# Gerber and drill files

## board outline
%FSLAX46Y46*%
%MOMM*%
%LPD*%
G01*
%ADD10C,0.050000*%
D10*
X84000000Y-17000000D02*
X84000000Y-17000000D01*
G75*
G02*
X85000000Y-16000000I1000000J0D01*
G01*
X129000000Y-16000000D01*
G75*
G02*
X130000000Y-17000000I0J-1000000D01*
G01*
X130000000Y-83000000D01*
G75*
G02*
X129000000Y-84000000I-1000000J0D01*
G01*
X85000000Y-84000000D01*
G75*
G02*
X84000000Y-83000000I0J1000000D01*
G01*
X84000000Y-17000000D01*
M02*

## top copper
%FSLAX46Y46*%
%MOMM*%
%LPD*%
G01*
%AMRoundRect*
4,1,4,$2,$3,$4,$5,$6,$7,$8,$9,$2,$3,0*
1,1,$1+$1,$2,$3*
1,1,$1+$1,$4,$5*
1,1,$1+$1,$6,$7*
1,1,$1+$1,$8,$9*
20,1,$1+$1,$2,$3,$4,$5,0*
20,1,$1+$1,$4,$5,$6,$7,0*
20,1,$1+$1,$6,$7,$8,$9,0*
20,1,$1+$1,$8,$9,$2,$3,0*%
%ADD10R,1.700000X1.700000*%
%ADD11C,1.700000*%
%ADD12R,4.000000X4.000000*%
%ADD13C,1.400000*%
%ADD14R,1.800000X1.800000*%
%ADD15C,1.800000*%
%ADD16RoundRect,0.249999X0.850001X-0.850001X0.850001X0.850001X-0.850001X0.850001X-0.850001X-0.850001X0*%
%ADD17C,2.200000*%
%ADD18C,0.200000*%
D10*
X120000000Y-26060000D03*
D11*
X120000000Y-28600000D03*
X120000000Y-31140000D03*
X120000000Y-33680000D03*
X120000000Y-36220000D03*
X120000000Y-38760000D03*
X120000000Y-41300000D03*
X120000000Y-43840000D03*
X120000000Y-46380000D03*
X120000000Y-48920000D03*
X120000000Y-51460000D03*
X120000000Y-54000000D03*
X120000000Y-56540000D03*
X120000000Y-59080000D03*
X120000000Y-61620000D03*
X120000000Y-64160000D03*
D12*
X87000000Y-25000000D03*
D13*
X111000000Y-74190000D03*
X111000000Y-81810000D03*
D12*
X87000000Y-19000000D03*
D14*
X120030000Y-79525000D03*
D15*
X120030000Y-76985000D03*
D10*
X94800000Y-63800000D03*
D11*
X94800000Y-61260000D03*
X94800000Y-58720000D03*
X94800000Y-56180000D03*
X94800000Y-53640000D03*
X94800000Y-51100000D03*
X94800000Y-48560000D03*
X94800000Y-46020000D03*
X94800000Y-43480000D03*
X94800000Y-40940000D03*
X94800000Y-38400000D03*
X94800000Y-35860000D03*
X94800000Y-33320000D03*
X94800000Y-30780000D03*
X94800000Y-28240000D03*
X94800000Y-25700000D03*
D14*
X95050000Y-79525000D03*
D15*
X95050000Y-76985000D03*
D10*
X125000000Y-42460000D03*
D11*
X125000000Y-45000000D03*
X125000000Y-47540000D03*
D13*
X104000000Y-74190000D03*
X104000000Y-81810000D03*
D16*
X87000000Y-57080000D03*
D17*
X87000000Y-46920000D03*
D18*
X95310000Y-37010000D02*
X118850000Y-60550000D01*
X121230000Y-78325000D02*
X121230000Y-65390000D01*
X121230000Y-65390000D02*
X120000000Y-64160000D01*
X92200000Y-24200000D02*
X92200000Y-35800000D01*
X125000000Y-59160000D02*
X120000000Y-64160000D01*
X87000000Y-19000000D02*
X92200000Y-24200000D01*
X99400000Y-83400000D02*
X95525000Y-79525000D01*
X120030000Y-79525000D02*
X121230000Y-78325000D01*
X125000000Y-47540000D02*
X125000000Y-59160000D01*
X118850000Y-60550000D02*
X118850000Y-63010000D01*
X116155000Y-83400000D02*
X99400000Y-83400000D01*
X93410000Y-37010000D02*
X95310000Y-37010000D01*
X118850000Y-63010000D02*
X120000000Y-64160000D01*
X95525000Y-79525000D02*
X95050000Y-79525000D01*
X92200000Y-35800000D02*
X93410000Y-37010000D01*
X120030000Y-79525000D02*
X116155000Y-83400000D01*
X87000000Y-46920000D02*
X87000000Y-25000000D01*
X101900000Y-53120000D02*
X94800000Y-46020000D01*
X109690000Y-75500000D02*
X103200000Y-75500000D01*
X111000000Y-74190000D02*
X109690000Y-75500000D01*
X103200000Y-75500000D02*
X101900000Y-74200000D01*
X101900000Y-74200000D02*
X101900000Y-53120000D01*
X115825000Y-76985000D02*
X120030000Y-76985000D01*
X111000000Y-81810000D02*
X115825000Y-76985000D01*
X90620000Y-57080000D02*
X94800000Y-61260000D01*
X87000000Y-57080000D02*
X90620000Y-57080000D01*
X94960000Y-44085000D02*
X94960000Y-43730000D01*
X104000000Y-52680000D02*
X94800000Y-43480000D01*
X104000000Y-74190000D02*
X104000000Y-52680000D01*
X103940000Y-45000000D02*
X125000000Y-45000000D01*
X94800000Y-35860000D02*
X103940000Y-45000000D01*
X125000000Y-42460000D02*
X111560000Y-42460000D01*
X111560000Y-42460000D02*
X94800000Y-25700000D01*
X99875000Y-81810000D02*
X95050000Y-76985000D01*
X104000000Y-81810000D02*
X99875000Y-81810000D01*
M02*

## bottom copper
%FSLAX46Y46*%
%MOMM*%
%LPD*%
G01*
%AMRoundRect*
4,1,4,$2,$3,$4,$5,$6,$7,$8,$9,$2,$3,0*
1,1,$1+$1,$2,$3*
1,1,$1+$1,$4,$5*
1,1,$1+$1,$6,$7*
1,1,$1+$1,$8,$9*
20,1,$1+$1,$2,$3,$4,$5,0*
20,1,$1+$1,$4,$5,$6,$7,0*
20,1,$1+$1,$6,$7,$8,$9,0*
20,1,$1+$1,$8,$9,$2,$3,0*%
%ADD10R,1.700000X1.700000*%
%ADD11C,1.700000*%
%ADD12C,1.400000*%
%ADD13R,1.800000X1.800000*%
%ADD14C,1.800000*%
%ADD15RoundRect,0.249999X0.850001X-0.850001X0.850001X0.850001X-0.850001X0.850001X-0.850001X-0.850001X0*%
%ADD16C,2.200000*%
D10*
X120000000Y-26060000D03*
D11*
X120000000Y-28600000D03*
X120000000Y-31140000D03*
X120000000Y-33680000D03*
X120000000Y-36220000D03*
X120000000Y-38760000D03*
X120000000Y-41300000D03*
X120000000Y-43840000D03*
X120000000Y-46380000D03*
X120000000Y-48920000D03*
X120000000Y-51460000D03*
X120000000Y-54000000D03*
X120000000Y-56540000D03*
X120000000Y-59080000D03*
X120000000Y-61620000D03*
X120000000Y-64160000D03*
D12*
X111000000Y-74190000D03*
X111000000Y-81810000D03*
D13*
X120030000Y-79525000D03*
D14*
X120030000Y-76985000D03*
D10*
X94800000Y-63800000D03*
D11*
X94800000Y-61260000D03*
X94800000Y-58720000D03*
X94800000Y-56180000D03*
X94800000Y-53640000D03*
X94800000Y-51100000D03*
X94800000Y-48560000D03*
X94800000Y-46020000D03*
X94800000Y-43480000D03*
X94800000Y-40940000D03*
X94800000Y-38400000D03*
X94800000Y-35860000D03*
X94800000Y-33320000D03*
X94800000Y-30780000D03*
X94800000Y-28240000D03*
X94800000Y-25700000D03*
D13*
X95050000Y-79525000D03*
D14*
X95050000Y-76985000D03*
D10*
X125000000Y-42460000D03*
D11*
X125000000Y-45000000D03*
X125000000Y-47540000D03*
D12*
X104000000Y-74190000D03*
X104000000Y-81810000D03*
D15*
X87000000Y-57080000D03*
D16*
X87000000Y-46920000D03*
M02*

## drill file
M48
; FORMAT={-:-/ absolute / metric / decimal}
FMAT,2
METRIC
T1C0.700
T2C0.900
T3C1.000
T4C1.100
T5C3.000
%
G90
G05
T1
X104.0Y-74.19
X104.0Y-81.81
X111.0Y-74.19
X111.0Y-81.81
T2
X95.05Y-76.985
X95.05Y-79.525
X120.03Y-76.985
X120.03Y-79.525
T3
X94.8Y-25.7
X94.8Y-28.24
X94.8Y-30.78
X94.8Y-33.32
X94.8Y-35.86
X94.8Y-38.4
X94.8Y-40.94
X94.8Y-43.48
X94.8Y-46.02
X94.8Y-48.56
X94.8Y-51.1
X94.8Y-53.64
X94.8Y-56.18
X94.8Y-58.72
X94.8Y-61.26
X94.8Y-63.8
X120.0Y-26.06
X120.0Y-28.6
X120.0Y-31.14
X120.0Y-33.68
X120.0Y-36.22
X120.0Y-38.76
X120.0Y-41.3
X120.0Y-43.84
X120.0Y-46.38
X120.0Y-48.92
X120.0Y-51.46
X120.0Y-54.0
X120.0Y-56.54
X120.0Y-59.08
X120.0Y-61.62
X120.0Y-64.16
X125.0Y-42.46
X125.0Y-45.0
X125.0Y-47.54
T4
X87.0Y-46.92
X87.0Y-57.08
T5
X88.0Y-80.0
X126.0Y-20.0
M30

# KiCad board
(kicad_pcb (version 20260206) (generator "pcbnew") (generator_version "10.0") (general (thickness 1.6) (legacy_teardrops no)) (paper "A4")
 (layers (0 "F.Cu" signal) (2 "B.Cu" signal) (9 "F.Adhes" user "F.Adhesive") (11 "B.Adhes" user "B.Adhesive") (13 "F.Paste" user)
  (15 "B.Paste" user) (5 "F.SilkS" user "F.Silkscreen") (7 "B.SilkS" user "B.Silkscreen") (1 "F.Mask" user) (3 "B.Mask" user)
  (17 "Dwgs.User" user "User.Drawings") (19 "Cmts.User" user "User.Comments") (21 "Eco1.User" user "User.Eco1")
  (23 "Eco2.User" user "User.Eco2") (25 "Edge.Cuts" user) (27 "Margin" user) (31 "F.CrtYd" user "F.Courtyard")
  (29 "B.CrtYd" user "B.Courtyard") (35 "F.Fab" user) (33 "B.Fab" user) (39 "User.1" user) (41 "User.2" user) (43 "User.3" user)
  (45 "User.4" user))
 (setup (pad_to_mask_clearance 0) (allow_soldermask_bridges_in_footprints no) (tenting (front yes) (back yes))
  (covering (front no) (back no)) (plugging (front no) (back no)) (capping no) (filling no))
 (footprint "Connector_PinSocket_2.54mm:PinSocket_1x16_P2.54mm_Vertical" (layer "F.Cu") (at 120 26.06)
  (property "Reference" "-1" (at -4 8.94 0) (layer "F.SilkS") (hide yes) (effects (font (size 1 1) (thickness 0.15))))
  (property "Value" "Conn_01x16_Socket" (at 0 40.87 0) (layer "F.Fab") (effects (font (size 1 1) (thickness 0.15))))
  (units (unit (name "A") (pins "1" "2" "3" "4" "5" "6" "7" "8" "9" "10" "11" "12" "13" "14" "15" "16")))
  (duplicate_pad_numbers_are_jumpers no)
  (pad "1" thru_hole rect (at 0 0) (size 1.7 1.7) (drill 1) (layers "*.Cu" "*.Mask") (remove_unused_layers no)
   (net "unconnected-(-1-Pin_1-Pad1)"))
  (pad "2" thru_hole circle (at 0 2.54) (size 1.7 1.7) (drill 1) (layers "*.Cu" "*.Mask") (remove_unused_layers no)
   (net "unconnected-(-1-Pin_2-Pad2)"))
  (pad "3" thru_hole circle (at 0 5.08) (size 1.7 1.7) (drill 1) (layers "*.Cu" "*.Mask") (remove_unused_layers no)
   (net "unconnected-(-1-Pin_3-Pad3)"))
  (pad "4" thru_hole circle (at 0 7.62) (size 1.7 1.7) (drill 1) (layers "*.Cu" "*.Mask") (remove_unused_layers no)
   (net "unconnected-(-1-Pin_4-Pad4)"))
  (pad "5" thru_hole circle (at 0 10.16) (size 1.7 1.7) (drill 1) (layers "*.Cu" "*.Mask") (remove_unused_layers no)
   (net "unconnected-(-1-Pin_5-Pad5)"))
  (pad "6" thru_hole circle (at 0 12.7) (size 1.7 1.7) (drill 1) (layers "*.Cu" "*.Mask") (remove_unused_layers no)
   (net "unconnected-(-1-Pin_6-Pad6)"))
  (pad "7" thru_hole circle (at 0 15.24) (size 1.7 1.7) (drill 1) (layers "*.Cu" "*.Mask") (remove_unused_layers no)
   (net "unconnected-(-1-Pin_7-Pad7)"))
  (pad "8" thru_hole circle (at 0 17.78) (size 1.7 1.7) (drill 1) (layers "*.Cu" "*.Mask") (remove_unused_layers no)
   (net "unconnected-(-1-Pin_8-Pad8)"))
  (pad "9" thru_hole circle (at 0 20.32) (size 1.7 1.7) (drill 1) (layers "*.Cu" "*.Mask") (remove_unused_layers no)
   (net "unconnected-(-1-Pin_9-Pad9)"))
  (pad "10" thru_hole circle (at 0 22.86) (size 1.7 1.7) (drill 1) (layers "*.Cu" "*.Mask") (remove_unused_layers no)
   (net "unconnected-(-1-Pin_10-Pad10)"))
  (pad "11" thru_hole circle (at 0 25.4) (size 1.7 1.7) (drill 1) (layers "*.Cu" "*.Mask") (remove_unused_layers no)
   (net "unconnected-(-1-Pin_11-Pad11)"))
  (pad "12" thru_hole circle (at 0 27.94) (size 1.7 1.7) (drill 1) (layers "*.Cu" "*.Mask") (remove_unused_layers no)
   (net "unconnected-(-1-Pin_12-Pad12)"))
  (pad "13" thru_hole circle (at 0 30.48) (size 1.7 1.7) (drill 1) (layers "*.Cu" "*.Mask") (remove_unused_layers no)
   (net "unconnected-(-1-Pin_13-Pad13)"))
  (pad "14" thru_hole circle (at 0 33.02) (size 1.7 1.7) (drill 1) (layers "*.Cu" "*.Mask") (remove_unused_layers no)
   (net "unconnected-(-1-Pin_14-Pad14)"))
  (pad "15" thru_hole circle (at 0 35.56) (size 1.7 1.7) (drill 1) (layers "*.Cu" "*.Mask") (remove_unused_layers no)
   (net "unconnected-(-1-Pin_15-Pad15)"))
  (pad "16" thru_hole circle (at 0 38.1) (size 1.7 1.7) (drill 1) (layers "*.Cu" "*.Mask") (remove_unused_layers no) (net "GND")))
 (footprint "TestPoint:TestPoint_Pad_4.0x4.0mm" (layer "F.Cu") (at 87 25)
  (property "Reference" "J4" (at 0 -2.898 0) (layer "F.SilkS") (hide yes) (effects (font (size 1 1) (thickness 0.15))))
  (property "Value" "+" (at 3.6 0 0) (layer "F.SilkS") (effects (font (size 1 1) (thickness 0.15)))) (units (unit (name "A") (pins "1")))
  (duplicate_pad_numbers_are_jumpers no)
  (pad "1" smd rect (at 0 0) (size 4 4) (layers "F.Cu" "F.Mask") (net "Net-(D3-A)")))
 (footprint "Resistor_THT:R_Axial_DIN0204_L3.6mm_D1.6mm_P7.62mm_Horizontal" (layer "F.Cu") (at 111 74.19 -90)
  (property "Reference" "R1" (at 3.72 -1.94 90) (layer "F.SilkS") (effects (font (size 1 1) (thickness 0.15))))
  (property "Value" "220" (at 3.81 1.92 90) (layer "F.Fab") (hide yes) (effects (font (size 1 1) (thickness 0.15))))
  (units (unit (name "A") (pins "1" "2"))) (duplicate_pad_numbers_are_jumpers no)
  (pad "1" thru_hole circle (at 0 0 270) (size 1.4 1.4) (drill 0.7) (layers "*.Cu" "*.Mask") (remove_unused_layers no) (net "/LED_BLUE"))
  (pad "2" thru_hole circle (at 7.62 0 270) (size 1.4 1.4) (drill 0.7) (layers "*.Cu" "*.Mask") (remove_unused_layers no) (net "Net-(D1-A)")))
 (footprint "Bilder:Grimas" (layer "F.Cu") (at 106 43)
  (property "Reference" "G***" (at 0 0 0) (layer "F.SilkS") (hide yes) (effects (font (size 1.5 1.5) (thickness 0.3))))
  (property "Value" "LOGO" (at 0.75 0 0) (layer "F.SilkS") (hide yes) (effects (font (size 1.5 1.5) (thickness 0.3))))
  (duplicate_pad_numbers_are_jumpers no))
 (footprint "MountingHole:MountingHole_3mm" (layer "F.Cu") (at 88 80)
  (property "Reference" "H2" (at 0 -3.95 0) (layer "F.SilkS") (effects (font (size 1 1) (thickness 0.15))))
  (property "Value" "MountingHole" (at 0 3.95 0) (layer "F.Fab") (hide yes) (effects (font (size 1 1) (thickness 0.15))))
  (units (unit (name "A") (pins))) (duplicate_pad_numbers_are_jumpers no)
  (pad "" np_thru_hole circle (at 0 0) (size 3 3) (drill 3) (layers "*.Cu" "*.Mask")))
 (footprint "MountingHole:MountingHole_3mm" (layer "F.Cu") (at 126 20)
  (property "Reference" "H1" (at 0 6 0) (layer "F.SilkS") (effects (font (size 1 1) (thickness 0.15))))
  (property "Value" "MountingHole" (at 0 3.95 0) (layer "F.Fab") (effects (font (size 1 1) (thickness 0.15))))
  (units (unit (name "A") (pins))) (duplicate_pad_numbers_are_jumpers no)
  (pad "" np_thru_hole circle (at 0 0) (size 3 3) (drill 3) (layers "*.Cu" "*.Mask")))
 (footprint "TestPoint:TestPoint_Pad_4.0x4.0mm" (layer "F.Cu") (at 87 19)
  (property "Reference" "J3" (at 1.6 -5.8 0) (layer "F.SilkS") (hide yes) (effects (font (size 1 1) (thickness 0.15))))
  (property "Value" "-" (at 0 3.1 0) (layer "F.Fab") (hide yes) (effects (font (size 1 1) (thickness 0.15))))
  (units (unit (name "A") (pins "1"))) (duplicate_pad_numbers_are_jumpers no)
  (pad "1" smd rect (at 0 0) (size 4 4) (layers "F.Cu" "F.Mask") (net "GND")))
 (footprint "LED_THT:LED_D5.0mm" (layer "F.Cu") (at 120.03 79.525 90)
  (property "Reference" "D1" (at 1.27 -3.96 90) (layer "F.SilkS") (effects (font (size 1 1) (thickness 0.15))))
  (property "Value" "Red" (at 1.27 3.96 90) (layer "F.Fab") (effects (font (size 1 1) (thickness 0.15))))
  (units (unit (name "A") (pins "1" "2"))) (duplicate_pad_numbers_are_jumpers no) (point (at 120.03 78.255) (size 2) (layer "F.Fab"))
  (pad "1" thru_hole rect (at 0 0 90) (size 1.8 1.8) (drill 0.9) (layers "*.Cu" "*.Mask") (remove_unused_layers no) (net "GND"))
  (pad "2" thru_hole circle (at 2.54 0 90) (size 1.8 1.8) (drill 0.9) (layers "*.Cu" "*.Mask") (remove_unused_layers no) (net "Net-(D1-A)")))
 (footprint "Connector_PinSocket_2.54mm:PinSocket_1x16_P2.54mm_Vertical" (layer "F.Cu") (at 94.8 63.8 180)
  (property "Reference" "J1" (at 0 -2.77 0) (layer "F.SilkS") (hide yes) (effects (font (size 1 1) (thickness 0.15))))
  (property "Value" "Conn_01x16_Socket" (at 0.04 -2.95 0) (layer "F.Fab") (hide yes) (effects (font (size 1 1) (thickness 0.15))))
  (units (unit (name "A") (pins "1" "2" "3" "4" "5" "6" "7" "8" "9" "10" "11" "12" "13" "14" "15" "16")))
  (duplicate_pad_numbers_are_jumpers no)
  (pad "1" thru_hole rect (at 0 0 180) (size 1.7 1.7) (drill 1) (layers "*.Cu" "*.Mask") (remove_unused_layers no)
   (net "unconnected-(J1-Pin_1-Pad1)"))
  (pad "2" thru_hole circle (at 0 2.54 180) (size 1.7 1.7) (drill 1) (layers "*.Cu" "*.Mask") (remove_unused_layers no) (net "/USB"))
  (pad "3" thru_hole circle (at 0 5.08 180) (size 1.7 1.7) (drill 1) (layers "*.Cu" "*.Mask") (remove_unused_layers no)
   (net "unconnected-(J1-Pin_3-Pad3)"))
  (pad "4" thru_hole circle (at 0 7.62 180) (size 1.7 1.7) (drill 1) (layers "*.Cu" "*.Mask") (remove_unused_layers no)
   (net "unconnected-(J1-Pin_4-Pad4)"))
  (pad "5" thru_hole circle (at 0 10.16 180) (size 1.7 1.7) (drill 1) (layers "*.Cu" "*.Mask") (remove_unused_layers no)
   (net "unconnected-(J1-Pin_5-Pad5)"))
  (pad "6" thru_hole circle (at 0 12.7 180) (size 1.7 1.7) (drill 1) (layers "*.Cu" "*.Mask") (remove_unused_layers no)
   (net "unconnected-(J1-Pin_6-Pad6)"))
  (pad "7" thru_hole circle (at 0 15.24 180) (size 1.7 1.7) (drill 1) (layers "*.Cu" "*.Mask") (remove_unused_layers no)
   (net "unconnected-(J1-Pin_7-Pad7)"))
  (pad "8" thru_hole circle (at 0 17.78 180) (size 1.7 1.7) (drill 1) (layers "*.Cu" "*.Mask") (remove_unused_layers no) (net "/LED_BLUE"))
  (pad "9" thru_hole circle (at 0 20.32 180) (size 1.7 1.7) (drill 1) (layers "*.Cu" "*.Mask") (remove_unused_layers no) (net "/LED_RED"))
  (pad "10" thru_hole circle (at 0 22.86 180) (size 1.7 1.7) (drill 1) (layers "*.Cu" "*.Mask") (remove_unused_layers no)
   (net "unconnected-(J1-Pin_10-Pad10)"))
  (pad "11" thru_hole circle (at 0 25.4 180) (size 1.7 1.7) (drill 1) (layers "*.Cu" "*.Mask") (remove_unused_layers no)
   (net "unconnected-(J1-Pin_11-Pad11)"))
  (pad "12" thru_hole circle (at 0 27.94 180) (size 1.7 1.7) (drill 1) (layers "*.Cu" "*.Mask") (remove_unused_layers no) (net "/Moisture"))
  (pad "13" thru_hole circle (at 0 30.48 180) (size 1.7 1.7) (drill 1) (layers "*.Cu" "*.Mask") (remove_unused_layers no)
   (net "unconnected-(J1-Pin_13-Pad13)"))
  (pad "14" thru_hole circle (at 0 33.02 180) (size 1.7 1.7) (drill 1) (layers "*.Cu" "*.Mask") (remove_unused_layers no)
   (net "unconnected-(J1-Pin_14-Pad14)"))
  (pad "15" thru_hole circle (at 0 35.56 180) (size 1.7 1.7) (drill 1) (layers "*.Cu" "*.Mask") (remove_unused_layers no)
   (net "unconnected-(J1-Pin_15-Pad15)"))
  (pad "16" thru_hole circle (at 0 38.1 180) (size 1.7 1.7) (drill 1) (layers "*.Cu" "*.Mask") (remove_unused_layers no) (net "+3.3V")))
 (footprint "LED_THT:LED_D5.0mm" (layer "F.Cu") (at 95.05 79.525 90)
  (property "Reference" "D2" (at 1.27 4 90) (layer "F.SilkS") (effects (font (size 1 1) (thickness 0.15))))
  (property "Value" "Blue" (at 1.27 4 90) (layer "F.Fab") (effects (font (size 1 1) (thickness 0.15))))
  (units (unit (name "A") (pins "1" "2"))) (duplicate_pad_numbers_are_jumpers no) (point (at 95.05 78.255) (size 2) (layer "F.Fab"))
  (pad "1" thru_hole rect (at 0 0 90) (size 1.8 1.8) (drill 0.9) (layers "*.Cu" "*.Mask") (remove_unused_layers no) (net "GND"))
  (pad "2" thru_hole circle (at 2.54 0 90) (size 1.8 1.8) (drill 0.9) (layers "*.Cu" "*.Mask") (remove_unused_layers no) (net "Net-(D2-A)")))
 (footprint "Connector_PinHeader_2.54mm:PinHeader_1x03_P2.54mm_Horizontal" (layer "F.Cu") (at 125 42.46)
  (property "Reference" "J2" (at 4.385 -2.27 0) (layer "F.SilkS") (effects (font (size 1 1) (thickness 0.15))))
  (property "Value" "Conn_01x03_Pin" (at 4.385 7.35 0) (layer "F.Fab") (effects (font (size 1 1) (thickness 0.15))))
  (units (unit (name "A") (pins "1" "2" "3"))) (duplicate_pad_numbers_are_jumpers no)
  (pad "1" thru_hole rect (at 0 0) (size 1.7 1.7) (drill 1) (layers "*.Cu" "*.Mask") (remove_unused_layers no) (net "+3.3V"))
  (pad "2" thru_hole circle (at 0 2.54) (size 1.7 1.7) (drill 1) (layers "*.Cu" "*.Mask") (remove_unused_layers no) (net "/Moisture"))
  (pad "3" thru_hole circle (at 0 5.08) (size 1.7 1.7) (drill 1) (layers "*.Cu" "*.Mask") (remove_unused_layers no) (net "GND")))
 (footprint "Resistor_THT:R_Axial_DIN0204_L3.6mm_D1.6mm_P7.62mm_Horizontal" (layer "F.Cu") (at 104 74.19 -90)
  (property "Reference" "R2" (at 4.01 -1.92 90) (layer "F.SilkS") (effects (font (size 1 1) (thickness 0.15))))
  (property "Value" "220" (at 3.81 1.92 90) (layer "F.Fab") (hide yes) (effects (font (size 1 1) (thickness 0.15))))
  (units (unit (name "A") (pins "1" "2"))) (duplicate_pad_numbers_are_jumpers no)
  (pad "1" thru_hole circle (at 0 0 270) (size 1.4 1.4) (drill 0.7) (layers "*.Cu" "*.Mask") (remove_unused_layers no) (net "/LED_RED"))
  (pad "2" thru_hole circle (at 7.62 0 270) (size 1.4 1.4) (drill 0.7) (layers "*.Cu" "*.Mask") (remove_unused_layers no) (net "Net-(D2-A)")))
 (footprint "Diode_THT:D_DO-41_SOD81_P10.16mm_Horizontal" (layer "F.Cu") (at 87 57.08 90)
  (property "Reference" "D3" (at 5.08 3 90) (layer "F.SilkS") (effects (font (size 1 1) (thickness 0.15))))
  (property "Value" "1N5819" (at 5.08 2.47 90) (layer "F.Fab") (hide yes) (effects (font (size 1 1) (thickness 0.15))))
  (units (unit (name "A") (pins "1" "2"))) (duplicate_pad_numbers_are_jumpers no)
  (pad "1" thru_hole roundrect (at 0 0 90) (size 2.2 2.2) (drill 1.1) (layers "*.Cu" "*.Mask") (remove_unused_layers no)
   (roundrect_rratio 0.113636) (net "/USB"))
  (pad "2" thru_hole circle (at 10.16 0 90) (size 2.2 2.2) (drill 1.1) (layers "*.Cu" "*.Mask") (remove_unused_layers no) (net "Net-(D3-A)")))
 (gr_rect (start 84 16) (end 130 84) (radius 1) (stroke (width 0.05) (type solid)) (fill no) (layer "Edge.Cuts"))
 (segment (start 95.31 37.01) (end 118.85 60.55) (width 0.2) (layer "F.Cu") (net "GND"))
 (segment (start 121.23 78.325) (end 121.23 65.39) (width 0.2) (layer "F.Cu") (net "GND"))
 (segment (start 121.23 65.39) (end 120 64.16) (width 0.2) (layer "F.Cu") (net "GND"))
 (segment (start 92.2 24.2) (end 92.2 35.8) (width 0.2) (layer "F.Cu") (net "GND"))
 (segment (start 125 59.16) (end 120 64.16) (width 0.2) (layer "F.Cu") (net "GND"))
 (segment (start 87 19) (end 92.2 24.2) (width 0.2) (layer "F.Cu") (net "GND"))
 (segment (start 99.4 83.4) (end 95.525 79.525) (width 0.2) (layer "F.Cu") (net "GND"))
 (segment (start 120.03 79.525) (end 121.23 78.325) (width 0.2) (layer "F.Cu") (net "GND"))
 (segment (start 125 47.54) (end 125 59.16) (width 0.2) (layer "F.Cu") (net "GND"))
 (segment (start 118.85 60.55) (end 118.85 63.01) (width 0.2) (layer "F.Cu") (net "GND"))
 (segment (start 116.155 83.4) (end 99.4 83.4) (width 0.2) (layer "F.Cu") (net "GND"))
 (segment (start 93.41 37.01) (end 95.31 37.01) (width 0.2) (layer "F.Cu") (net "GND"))
 (segment (start 118.85 63.01) (end 120 64.16) (width 0.2) (layer "F.Cu") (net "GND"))
 (segment (start 95.525 79.525) (end 95.05 79.525) (width 0.2) (layer "F.Cu") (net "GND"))
 (segment (start 92.2 35.8) (end 93.41 37.01) (width 0.2) (layer "F.Cu") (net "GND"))
 (segment (start 120.03 79.525) (end 116.155 83.4) (width 0.2) (layer "F.Cu") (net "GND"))
 (segment (start 87 46.92) (end 87 25) (width 0.2) (layer "F.Cu") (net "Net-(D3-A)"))
 (segment (start 101.9 53.12) (end 94.8 46.02) (width 0.2) (layer "F.Cu") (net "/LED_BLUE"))
 (segment (start 109.69 75.5) (end 103.2 75.5) (width 0.2) (layer "F.Cu") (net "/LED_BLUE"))
 (segment (start 111 74.19) (end 109.69 75.5) (width 0.2) (layer "F.Cu") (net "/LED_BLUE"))
 (segment (start 103.2 75.5) (end 101.9 74.2) (width 0.2) (layer "F.Cu") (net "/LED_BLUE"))
 (segment (start 101.9 74.2) (end 101.9 53.12) (width 0.2) (layer "F.Cu") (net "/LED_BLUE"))
 (segment (start 115.825 76.985) (end 120.03 76.985) (width 0.2) (layer "F.Cu") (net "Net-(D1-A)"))
 (segment (start 111 81.81) (end 115.825 76.985) (width 0.2) (layer "F.Cu") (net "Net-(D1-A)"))
 (segment (start 90.62 57.08) (end 94.8 61.26) (width 0.2) (layer "F.Cu") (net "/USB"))
 (segment (start 87 57.08) (end 90.62 57.08) (width 0.2) (layer "F.Cu") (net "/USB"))
 (segment (start 94.96 44.085) (end 94.96 43.73) (width 0.2) (layer "F.Cu") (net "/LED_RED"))
 (segment (start 104 52.68) (end 94.8 43.48) (width 0.2) (layer "F.Cu") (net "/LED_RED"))
 (segment (start 104 74.19) (end 104 52.68) (width 0.2) (layer "F.Cu") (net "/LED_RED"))
 (segment (start 103.94 45) (end 125 45) (width 0.2) (layer "F.Cu") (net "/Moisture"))
 (segment (start 94.8 35.86) (end 103.94 45) (width 0.2) (layer "F.Cu") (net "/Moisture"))
 (segment (start 125 42.46) (end 111.56 42.46) (width 0.2) (layer "F.Cu") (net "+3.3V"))
 (segment (start 111.56 42.46) (end 94.8 25.7) (width 0.2) (layer "F.Cu") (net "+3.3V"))
 (segment (start 99.875 81.81) (end 95.05 76.985) (width 0.2) (layer "F.Cu") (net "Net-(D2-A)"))
 (segment (start 104 81.81) (end 99.875 81.81) (width 0.2) (layer "F.Cu") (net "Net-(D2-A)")))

